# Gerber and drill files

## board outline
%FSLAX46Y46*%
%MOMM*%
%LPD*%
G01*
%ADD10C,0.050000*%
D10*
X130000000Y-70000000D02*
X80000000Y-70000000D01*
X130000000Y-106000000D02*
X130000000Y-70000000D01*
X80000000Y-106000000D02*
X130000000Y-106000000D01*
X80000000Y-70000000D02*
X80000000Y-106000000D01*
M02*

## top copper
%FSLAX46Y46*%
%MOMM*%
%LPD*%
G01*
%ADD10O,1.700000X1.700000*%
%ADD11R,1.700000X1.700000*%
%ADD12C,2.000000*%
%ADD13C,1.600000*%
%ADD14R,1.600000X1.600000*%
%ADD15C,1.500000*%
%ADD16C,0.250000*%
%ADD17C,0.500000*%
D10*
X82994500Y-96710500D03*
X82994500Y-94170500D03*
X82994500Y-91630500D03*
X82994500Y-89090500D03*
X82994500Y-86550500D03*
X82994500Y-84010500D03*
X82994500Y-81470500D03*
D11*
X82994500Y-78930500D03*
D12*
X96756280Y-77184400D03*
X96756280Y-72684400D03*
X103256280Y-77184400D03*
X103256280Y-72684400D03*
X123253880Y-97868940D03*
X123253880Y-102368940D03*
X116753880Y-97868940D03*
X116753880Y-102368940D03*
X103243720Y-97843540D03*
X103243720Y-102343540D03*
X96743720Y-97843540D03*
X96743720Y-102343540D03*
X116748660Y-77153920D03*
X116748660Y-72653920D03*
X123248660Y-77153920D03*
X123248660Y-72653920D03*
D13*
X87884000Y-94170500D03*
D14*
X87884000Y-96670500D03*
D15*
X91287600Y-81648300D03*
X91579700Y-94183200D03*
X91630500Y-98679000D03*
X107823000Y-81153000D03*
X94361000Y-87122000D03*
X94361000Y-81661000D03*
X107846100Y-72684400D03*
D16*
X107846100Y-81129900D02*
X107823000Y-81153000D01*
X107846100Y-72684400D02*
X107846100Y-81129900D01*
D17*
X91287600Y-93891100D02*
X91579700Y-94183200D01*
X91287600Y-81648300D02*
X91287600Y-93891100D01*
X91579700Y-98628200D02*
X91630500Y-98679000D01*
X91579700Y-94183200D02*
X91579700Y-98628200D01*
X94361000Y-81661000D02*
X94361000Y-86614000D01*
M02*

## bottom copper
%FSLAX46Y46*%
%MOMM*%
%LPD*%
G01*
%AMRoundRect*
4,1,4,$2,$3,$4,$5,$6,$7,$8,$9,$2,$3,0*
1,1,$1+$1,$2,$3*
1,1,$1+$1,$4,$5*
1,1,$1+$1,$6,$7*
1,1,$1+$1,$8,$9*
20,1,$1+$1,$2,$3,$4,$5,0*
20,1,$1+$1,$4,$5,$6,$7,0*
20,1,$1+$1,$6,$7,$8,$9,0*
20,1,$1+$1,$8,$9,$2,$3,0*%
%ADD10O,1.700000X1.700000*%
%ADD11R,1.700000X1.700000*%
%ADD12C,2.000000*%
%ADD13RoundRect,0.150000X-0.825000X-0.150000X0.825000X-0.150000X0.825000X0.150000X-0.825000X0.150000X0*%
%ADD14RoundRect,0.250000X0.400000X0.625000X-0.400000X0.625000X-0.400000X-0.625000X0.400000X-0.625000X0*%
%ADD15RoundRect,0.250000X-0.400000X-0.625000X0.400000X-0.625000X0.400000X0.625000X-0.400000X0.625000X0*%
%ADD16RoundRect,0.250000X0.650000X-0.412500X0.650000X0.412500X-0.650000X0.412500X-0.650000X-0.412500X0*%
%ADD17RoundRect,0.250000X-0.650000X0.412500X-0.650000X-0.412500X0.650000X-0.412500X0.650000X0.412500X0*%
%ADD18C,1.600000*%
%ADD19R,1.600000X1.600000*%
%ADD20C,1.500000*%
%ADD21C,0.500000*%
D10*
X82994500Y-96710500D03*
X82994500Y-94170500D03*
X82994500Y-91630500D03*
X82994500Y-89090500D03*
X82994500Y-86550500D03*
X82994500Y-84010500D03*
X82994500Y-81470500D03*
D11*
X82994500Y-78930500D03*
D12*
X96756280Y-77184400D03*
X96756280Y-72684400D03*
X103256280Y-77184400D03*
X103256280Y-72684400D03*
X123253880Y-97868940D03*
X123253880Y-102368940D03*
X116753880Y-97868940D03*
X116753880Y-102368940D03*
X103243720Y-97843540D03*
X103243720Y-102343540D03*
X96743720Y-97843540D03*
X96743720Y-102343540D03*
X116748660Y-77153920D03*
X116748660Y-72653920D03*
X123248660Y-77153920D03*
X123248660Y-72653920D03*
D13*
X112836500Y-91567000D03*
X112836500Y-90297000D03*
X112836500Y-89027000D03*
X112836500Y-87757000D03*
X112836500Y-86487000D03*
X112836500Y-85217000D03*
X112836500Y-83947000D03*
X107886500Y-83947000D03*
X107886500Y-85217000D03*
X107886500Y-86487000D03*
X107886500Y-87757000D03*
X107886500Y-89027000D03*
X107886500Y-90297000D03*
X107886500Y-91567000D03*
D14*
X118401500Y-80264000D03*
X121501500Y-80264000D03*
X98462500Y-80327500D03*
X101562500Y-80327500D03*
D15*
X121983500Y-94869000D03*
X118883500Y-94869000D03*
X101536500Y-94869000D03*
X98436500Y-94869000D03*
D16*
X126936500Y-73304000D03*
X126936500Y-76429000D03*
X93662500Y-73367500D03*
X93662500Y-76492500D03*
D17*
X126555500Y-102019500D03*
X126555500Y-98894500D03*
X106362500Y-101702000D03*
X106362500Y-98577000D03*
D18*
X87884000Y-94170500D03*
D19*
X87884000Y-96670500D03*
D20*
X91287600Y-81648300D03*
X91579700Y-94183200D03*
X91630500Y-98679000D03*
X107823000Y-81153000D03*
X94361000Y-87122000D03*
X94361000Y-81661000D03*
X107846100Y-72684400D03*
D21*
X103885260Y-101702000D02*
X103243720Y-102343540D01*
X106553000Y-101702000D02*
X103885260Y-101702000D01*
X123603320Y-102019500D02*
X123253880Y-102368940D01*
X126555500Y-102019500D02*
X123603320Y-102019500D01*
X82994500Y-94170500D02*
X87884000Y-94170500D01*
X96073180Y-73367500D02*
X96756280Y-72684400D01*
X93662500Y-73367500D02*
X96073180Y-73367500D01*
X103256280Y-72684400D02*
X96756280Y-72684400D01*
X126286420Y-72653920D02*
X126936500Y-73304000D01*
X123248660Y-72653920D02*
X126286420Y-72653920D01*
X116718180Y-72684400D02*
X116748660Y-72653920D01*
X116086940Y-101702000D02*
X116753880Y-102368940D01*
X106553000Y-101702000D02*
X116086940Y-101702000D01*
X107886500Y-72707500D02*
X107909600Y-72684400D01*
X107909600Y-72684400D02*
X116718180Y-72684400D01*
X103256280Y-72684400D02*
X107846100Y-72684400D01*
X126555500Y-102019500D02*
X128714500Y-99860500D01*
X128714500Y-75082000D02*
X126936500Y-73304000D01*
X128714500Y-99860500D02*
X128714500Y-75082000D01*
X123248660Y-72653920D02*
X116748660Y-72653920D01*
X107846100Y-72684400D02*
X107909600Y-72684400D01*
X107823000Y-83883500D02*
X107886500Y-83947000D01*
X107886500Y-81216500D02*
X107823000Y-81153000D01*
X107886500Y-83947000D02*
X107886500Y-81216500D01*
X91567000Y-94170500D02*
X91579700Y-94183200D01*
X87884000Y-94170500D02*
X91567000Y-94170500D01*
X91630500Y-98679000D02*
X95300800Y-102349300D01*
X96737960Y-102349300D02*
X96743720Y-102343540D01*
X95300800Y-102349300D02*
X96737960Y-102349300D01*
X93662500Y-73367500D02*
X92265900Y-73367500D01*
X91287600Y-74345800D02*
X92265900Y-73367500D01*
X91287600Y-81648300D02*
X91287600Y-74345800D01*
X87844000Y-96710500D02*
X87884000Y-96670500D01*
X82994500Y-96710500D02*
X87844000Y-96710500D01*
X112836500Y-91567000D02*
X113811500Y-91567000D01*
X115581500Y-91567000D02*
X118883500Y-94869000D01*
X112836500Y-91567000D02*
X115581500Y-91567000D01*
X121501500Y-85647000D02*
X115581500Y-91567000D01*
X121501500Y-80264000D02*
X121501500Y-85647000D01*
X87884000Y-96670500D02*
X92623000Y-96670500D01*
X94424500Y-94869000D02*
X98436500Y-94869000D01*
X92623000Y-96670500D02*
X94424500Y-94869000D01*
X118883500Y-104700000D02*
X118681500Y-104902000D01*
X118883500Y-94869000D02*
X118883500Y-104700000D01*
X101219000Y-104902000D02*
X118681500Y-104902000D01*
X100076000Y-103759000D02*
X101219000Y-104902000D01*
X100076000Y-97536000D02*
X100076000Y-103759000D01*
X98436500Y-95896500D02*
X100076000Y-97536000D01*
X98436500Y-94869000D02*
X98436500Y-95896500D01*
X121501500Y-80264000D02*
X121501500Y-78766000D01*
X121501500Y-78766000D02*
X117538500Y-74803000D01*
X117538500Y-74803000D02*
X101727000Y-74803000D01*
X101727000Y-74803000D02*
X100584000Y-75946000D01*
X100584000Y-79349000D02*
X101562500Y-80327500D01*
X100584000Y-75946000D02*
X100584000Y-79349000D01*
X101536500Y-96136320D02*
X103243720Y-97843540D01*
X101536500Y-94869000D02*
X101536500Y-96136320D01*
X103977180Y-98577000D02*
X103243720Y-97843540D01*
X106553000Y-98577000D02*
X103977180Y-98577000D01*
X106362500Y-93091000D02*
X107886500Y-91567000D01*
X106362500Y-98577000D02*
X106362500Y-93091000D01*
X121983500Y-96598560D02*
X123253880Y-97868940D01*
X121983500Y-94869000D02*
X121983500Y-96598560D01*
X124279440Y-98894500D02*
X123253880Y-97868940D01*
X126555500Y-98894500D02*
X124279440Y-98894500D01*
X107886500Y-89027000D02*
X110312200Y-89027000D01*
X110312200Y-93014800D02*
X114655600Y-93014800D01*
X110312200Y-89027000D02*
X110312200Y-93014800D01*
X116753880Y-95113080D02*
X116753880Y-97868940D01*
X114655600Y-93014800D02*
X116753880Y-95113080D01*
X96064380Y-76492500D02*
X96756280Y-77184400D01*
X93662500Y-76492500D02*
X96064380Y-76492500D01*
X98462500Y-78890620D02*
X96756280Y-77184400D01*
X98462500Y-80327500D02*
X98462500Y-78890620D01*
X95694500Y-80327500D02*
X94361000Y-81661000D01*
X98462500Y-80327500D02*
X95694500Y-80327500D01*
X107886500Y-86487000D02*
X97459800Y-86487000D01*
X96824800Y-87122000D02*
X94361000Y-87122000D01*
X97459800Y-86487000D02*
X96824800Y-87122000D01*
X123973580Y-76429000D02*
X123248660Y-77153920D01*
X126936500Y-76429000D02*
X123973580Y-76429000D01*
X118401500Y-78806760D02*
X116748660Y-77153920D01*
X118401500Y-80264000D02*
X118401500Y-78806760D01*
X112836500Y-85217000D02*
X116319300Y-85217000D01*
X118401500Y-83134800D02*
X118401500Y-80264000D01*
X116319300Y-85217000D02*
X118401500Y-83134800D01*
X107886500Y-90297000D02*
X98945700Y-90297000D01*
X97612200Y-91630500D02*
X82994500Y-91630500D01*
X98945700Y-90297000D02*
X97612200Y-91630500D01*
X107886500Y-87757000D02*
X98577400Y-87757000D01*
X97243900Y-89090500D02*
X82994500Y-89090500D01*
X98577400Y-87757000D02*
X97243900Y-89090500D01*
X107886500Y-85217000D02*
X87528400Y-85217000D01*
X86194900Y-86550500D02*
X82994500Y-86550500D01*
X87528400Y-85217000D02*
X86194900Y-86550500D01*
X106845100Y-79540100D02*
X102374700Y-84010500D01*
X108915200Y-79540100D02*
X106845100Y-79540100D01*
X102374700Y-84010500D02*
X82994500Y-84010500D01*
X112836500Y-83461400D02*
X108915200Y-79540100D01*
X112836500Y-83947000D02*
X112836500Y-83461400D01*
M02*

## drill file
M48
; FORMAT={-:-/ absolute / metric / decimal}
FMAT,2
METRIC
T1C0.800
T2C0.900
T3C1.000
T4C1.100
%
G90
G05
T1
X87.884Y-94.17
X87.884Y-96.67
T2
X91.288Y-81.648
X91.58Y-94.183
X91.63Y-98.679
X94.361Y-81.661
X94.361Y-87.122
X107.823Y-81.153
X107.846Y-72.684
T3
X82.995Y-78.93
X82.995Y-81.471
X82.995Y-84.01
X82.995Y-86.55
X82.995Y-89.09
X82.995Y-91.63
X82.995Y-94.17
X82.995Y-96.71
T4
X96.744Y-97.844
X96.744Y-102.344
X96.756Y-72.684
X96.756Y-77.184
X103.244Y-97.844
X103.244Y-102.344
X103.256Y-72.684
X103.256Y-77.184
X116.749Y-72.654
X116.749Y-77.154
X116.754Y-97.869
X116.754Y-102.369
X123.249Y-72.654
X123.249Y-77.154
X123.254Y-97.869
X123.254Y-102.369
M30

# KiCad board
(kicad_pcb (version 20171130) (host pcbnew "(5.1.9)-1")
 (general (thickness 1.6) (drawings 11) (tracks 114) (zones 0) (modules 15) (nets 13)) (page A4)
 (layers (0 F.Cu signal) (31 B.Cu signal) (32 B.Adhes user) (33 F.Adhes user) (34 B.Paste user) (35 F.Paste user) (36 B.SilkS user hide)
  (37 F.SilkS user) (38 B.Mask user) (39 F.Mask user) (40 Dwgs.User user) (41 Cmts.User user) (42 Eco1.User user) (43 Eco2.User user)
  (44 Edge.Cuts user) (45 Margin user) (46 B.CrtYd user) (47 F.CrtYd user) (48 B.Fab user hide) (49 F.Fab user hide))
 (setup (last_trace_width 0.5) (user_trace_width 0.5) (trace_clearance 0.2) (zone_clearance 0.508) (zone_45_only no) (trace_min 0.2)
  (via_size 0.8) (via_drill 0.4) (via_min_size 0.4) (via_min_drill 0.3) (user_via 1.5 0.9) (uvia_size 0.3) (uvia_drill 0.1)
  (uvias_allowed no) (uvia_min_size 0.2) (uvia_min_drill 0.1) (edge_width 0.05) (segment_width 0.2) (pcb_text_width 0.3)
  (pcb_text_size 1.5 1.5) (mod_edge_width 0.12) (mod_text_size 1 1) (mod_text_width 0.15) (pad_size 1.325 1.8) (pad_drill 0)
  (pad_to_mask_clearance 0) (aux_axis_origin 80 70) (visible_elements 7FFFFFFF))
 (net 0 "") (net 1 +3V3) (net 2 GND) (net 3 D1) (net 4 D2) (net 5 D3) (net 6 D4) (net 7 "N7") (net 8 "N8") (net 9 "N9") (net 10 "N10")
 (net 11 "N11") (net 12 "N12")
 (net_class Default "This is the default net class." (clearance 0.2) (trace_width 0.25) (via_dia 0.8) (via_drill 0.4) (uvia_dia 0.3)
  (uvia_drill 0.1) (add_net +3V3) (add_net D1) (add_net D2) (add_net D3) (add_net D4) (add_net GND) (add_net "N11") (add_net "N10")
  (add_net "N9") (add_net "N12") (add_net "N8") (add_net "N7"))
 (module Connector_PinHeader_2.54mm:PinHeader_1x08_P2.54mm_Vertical (layer F.Cu) (at 82.9945 78.9305)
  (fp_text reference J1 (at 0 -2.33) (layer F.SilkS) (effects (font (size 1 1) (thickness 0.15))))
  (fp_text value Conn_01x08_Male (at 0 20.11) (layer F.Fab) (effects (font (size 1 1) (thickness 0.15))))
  (pad 8 thru_hole oval (at 0 17.78) (size 1.7 1.7) (drill 1) (layers *.Cu *.Mask) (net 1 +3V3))
  (pad 7 thru_hole oval (at 0 15.24) (size 1.7 1.7) (drill 1) (layers *.Cu *.Mask) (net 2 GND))
  (pad 6 thru_hole oval (at 0 12.7) (size 1.7 1.7) (drill 1) (layers *.Cu *.Mask) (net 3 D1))
  (pad 5 thru_hole oval (at 0 10.16) (size 1.7 1.7) (drill 1) (layers *.Cu *.Mask) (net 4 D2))
  (pad 4 thru_hole oval (at 0 7.62) (size 1.7 1.7) (drill 1) (layers *.Cu *.Mask) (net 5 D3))
  (pad 3 thru_hole oval (at 0 5.08) (size 1.7 1.7) (drill 1) (layers *.Cu *.Mask) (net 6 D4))
  (pad 2 thru_hole oval (at 0 2.54) (size 1.7 1.7) (drill 1) (layers *.Cu *.Mask) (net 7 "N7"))
  (pad 1 thru_hole rect (at 0 0) (size 1.7 1.7) (drill 1) (layers *.Cu *.Mask) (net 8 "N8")))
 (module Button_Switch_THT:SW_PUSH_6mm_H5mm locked (layer F.Cu) (at 100 75 180)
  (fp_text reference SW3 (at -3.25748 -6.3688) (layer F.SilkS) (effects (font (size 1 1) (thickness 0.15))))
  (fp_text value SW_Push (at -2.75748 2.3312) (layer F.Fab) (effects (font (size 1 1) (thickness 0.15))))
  (pad 1 thru_hole circle (at 3.24372 -2.1844 270) (size 2 2) (drill 1.1) (layers *.Cu *.Mask) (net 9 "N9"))
  (pad 2 thru_hole circle (at 3.24372 2.3156 270) (size 2 2) (drill 1.1) (layers *.Cu *.Mask) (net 2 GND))
  (pad 1 thru_hole circle (at -3.25628 -2.1844 270) (size 2 2) (drill 1.1) (layers *.Cu *.Mask) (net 9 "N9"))
  (pad 2 thru_hole circle (at -3.25628 2.3156 270) (size 2 2) (drill 1.1) (layers *.Cu *.Mask) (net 2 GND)))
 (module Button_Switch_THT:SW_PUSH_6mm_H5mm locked (layer F.Cu) (at 120 100)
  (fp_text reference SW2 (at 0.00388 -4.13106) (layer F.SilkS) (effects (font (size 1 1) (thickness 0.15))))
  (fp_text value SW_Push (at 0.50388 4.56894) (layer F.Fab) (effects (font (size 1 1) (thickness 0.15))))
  (pad 1 thru_hole circle (at 3.25388 -2.13106 90) (size 2 2) (drill 1.1) (layers *.Cu *.Mask) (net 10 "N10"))
  (pad 2 thru_hole circle (at 3.25388 2.36894 90) (size 2 2) (drill 1.1) (layers *.Cu *.Mask) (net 2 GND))
  (pad 1 thru_hole circle (at -3.24612 -2.13106 90) (size 2 2) (drill 1.1) (layers *.Cu *.Mask) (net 10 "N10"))
  (pad 2 thru_hole circle (at -3.24612 2.36894 90) (size 2 2) (drill 1.1) (layers *.Cu *.Mask) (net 2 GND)))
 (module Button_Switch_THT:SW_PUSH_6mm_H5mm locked (layer F.Cu) (at 100 100)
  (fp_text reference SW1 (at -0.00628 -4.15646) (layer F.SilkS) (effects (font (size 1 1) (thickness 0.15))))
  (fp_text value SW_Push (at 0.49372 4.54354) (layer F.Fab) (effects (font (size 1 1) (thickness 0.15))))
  (pad 1 thru_hole circle (at 3.24372 -2.15646 90) (size 2 2) (drill 1.1) (layers *.Cu *.Mask) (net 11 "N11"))
  (pad 2 thru_hole circle (at 3.24372 2.34354 90) (size 2 2) (drill 1.1) (layers *.Cu *.Mask) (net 2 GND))
  (pad 1 thru_hole circle (at -3.25628 -2.15646 90) (size 2 2) (drill 1.1) (layers *.Cu *.Mask) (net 11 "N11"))
  (pad 2 thru_hole circle (at -3.25628 2.34354 90) (size 2 2) (drill 1.1) (layers *.Cu *.Mask) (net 2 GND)))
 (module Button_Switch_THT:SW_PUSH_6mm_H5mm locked (layer F.Cu) (at 120 75 180)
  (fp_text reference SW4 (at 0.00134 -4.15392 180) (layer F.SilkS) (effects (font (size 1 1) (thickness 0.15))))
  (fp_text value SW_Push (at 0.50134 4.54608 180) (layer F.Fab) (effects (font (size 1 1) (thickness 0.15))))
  (pad 1 thru_hole circle (at 3.25134 -2.15392 270) (size 2 2) (drill 1.1) (layers *.Cu *.Mask) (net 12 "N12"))
  (pad 2 thru_hole circle (at 3.25134 2.34608 270) (size 2 2) (drill 1.1) (layers *.Cu *.Mask) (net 2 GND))
  (pad 1 thru_hole circle (at -3.24866 -2.15392 270) (size 2 2) (drill 1.1) (layers *.Cu *.Mask) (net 12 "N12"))
  (pad 2 thru_hole circle (at -3.24866 2.34608 270) (size 2 2) (drill 1.1) (layers *.Cu *.Mask) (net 2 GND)))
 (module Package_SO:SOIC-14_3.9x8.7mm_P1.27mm (layer B.Cu) (at 110.3615 87.757)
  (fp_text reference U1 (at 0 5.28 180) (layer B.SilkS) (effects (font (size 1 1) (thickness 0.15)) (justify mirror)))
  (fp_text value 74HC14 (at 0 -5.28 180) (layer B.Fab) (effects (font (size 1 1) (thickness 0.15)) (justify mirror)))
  (pad 14 smd roundrect (at 2.475 3.81) (size 1.95 0.6) (layers B.Cu B.Paste B.Mask) (roundrect_rratio 0.25) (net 1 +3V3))
  (pad 13 smd roundrect (at 2.475 2.54) (size 1.95 0.6) (layers B.Cu B.Paste B.Mask) (roundrect_rratio 0.25))
  (pad 12 smd roundrect (at 2.475 1.27) (size 1.95 0.6) (layers B.Cu B.Paste B.Mask) (roundrect_rratio 0.25))
  (pad 11 smd roundrect (at 2.475 0) (size 1.95 0.6) (layers B.Cu B.Paste B.Mask) (roundrect_rratio 0.25))
  (pad 10 smd roundrect (at 2.475 -1.27) (size 1.95 0.6) (layers B.Cu B.Paste B.Mask) (roundrect_rratio 0.25))
  (pad 9 smd roundrect (at 2.475 -2.54) (size 1.95 0.6) (layers B.Cu B.Paste B.Mask) (roundrect_rratio 0.25) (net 12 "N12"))
  (pad 8 smd roundrect (at 2.475 -3.81) (size 1.95 0.6) (layers B.Cu B.Paste B.Mask) (roundrect_rratio 0.25) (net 6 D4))
  (pad 7 smd roundrect (at -2.475 -3.81) (size 1.95 0.6) (layers B.Cu B.Paste B.Mask) (roundrect_rratio 0.25) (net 2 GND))
  (pad 6 smd roundrect (at -2.475 -2.54) (size 1.95 0.6) (layers B.Cu B.Paste B.Mask) (roundrect_rratio 0.25) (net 5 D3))
  (pad 5 smd roundrect (at -2.475 -1.27) (size 1.95 0.6) (layers B.Cu B.Paste B.Mask) (roundrect_rratio 0.25) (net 9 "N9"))
  (pad 4 smd roundrect (at -2.475 0) (size 1.95 0.6) (layers B.Cu B.Paste B.Mask) (roundrect_rratio 0.25) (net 4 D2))
  (pad 3 smd roundrect (at -2.475 1.27) (size 1.95 0.6) (layers B.Cu B.Paste B.Mask) (roundrect_rratio 0.25) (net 10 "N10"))
  (pad 2 smd roundrect (at -2.475 2.54) (size 1.95 0.6) (layers B.Cu B.Paste B.Mask) (roundrect_rratio 0.25) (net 3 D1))
  (pad 1 smd roundrect (at -2.475 3.81) (size 1.95 0.6) (layers B.Cu B.Paste B.Mask) (roundrect_rratio 0.25) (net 11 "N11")))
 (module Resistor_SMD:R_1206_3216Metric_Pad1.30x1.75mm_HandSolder (layer B.Cu) (at 119.9515 80.264 180)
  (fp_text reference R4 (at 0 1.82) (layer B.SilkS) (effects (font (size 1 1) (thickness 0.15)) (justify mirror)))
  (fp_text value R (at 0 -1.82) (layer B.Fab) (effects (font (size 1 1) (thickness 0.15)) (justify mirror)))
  (pad 2 smd roundrect (at 1.55 0 180) (size 1.3 1.75) (layers B.Cu B.Paste B.Mask) (roundrect_rratio 0.192308) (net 12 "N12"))
  (pad 1 smd roundrect (at -1.55 0 180) (size 1.3 1.75) (layers B.Cu B.Paste B.Mask) (roundrect_rratio 0.192308) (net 1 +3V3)))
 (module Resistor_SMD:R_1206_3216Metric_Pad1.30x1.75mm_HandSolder (layer B.Cu) (at 100.0125 80.3275 180)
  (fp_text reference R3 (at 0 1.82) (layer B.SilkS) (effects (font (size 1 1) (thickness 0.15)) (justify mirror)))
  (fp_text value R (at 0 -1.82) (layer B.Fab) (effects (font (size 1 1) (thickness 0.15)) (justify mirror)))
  (pad 2 smd roundrect (at 1.55 0 180) (size 1.3 1.75) (layers B.Cu B.Paste B.Mask) (roundrect_rratio 0.192308) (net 9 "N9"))
  (pad 1 smd roundrect (at -1.55 0 180) (size 1.3 1.75) (layers B.Cu B.Paste B.Mask) (roundrect_rratio 0.192308) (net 1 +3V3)))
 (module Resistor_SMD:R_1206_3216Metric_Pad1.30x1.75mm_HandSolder (layer B.Cu) (at 120.4335 94.869)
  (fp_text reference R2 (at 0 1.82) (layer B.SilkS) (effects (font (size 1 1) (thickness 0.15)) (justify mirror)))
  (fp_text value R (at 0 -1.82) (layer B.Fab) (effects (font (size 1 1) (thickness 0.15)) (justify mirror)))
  (pad 2 smd roundrect (at 1.55 0) (size 1.3 1.75) (layers B.Cu B.Paste B.Mask) (roundrect_rratio 0.192308) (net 10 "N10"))
  (pad 1 smd roundrect (at -1.55 0) (size 1.3 1.75) (layers B.Cu B.Paste B.Mask) (roundrect_rratio 0.192308) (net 1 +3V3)))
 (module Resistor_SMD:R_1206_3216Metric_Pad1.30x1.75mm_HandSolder (layer B.Cu) (at 99.9865 94.869)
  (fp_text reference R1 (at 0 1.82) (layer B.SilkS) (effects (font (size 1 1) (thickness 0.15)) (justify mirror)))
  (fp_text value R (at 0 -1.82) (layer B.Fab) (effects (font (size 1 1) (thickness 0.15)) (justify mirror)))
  (pad 2 smd roundrect (at 1.55 0) (size 1.3 1.75) (layers B.Cu B.Paste B.Mask) (roundrect_rratio 0.192308) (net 11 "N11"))
  (pad 1 smd roundrect (at -1.55 0) (size 1.3 1.75) (layers B.Cu B.Paste B.Mask) (roundrect_rratio 0.192308) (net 1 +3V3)))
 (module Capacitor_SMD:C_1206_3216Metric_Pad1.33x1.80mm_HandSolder (layer B.Cu) (at 126.9365 74.8665 90)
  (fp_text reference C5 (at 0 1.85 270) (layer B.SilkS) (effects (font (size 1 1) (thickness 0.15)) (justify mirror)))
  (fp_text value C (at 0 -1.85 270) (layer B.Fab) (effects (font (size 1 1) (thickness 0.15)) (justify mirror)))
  (pad 2 smd roundrect (at 1.5625 0 90) (size 1.325 1.8) (layers B.Cu B.Paste B.Mask) (roundrect_rratio 0.188679) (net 2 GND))
  (pad 1 smd roundrect (at -1.5625 0 90) (size 1.325 1.8) (layers B.Cu B.Paste B.Mask) (roundrect_rratio 0.188679) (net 12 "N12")))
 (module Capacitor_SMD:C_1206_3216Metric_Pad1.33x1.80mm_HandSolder (layer B.Cu) (at 93.6625 74.93 90)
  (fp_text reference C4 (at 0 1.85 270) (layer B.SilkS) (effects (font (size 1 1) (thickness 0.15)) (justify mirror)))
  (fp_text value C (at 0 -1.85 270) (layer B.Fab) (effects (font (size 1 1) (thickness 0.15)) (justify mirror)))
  (pad 2 smd roundrect (at 1.5625 0 90) (size 1.325 1.8) (layers B.Cu B.Paste B.Mask) (roundrect_rratio 0.188679) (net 2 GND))
  (pad 1 smd roundrect (at -1.5625 0 90) (size 1.325 1.8) (layers B.Cu B.Paste B.Mask) (roundrect_rratio 0.188679) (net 9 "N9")))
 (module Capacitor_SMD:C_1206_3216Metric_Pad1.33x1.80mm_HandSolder (layer B.Cu) (at 126.5555 100.457 270)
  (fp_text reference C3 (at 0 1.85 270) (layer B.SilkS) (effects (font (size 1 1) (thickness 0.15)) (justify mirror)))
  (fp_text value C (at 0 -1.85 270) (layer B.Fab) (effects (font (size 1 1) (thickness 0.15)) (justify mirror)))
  (pad 2 smd roundrect (at 1.5625 0 270) (size 1.325 1.8) (layers B.Cu B.Paste B.Mask) (roundrect_rratio 0.188679) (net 2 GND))
  (pad 1 smd roundrect (at -1.5625 0 270) (size 1.325 1.8) (layers B.Cu B.Paste B.Mask) (roundrect_rratio 0.188679) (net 10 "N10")))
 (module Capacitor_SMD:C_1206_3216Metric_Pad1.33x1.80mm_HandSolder (layer B.Cu) (at 106.3625 100.1395 270)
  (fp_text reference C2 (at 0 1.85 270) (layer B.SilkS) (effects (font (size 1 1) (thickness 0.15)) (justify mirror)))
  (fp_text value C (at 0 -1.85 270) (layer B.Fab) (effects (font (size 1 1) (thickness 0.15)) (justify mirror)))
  (pad 2 smd roundrect (at 1.5625 0 270) (size 1.325 1.8) (layers B.Cu B.Paste B.Mask) (roundrect_rratio 0.188679) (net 2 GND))
  (pad 1 smd roundrect (at -1.5625 0 270) (size 1.325 1.8) (layers B.Cu B.Paste B.Mask) (roundrect_rratio 0.188679) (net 11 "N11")))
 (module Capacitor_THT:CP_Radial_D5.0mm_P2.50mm (layer F.Cu) (at 87.884 96.6705 90)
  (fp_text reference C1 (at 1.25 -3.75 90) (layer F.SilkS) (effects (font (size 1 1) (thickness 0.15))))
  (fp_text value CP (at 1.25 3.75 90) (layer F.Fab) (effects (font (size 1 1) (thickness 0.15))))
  (pad 2 thru_hole circle (at 2.5 0 90) (size 1.6 1.6) (drill 0.8) (layers *.Cu *.Mask) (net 2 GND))
  (pad 1 thru_hole rect (at 0 0 90) (size 1.6 1.6) (drill 0.8) (layers *.Cu *.Mask) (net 1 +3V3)))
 (gr_line (start 130 70) (end 80 70) (layer Edge.Cuts) (width 0.05))
 (gr_line (start 130 106) (end 130 70) (layer Edge.Cuts) (width 0.05))
 (gr_line (start 80 106) (end 130 106) (layer Edge.Cuts) (width 0.05))
 (gr_line (start 80 70) (end 80 106) (layer Edge.Cuts) (width 0.05))
 (via (at 91.2876 81.6483) (size 1.5) (drill 0.9) (layers F.Cu B.Cu) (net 2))
 (via (at 91.5797 94.1832) (size 1.5) (drill 0.9) (layers F.Cu B.Cu) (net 2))
 (via (at 91.6305 98.679) (size 1.5) (drill 0.9) (layers F.Cu B.Cu) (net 2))
 (via (at 107.823 81.153) (size 1.5) (drill 0.9) (layers F.Cu B.Cu) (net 2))
 (via (at 94.361 87.122) (size 1.5) (drill 0.9) (layers F.Cu B.Cu) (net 9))
 (via (at 94.361 81.661) (size 1.5) (drill 0.9) (layers F.Cu B.Cu) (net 9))
 (segment (start 103.88526 101.702) (end 103.24372 102.34354) (width 0.5) (layer B.Cu) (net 2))
 (segment (start 106.553 101.702) (end 103.88526 101.702) (width 0.5) (layer B.Cu) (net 2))
 (segment (start 123.60332 102.0195) (end 123.25388 102.36894) (width 0.5) (layer B.Cu) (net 2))
 (segment (start 126.5555 102.0195) (end 123.60332 102.0195) (width 0.5) (layer B.Cu) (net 2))
 (segment (start 82.9945 94.1705) (end 87.884 94.1705) (width 0.5) (layer B.Cu) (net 2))
 (segment (start 96.07318 73.3675) (end 96.75628 72.6844) (width 0.5) (layer B.Cu) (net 2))
 (segment (start 93.6625 73.3675) (end 96.07318 73.3675) (width 0.5) (layer B.Cu) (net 2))
 (segment (start 103.25628 72.6844) (end 96.75628 72.6844) (width 0.5) (layer B.Cu) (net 2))
 (segment (start 126.28642 72.65392) (end 126.9365 73.304) (width 0.5) (layer B.Cu) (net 2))
 (segment (start 123.24866 72.65392) (end 126.28642 72.65392) (width 0.5) (layer B.Cu) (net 2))
 (segment (start 116.71818 72.6844) (end 116.74866 72.65392) (width 0.5) (layer B.Cu) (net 2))
 (segment (start 116.08694 101.702) (end 116.75388 102.36894) (width 0.5) (layer B.Cu) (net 2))
 (segment (start 106.553 101.702) (end 116.08694 101.702) (width 0.5) (layer B.Cu) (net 2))
 (segment (start 107.8865 72.7075) (end 107.9096 72.6844) (width 0.5) (layer B.Cu) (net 2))
 (segment (start 107.9096 72.6844) (end 116.71818 72.6844) (width 0.5) (layer B.Cu) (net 2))
 (segment (start 103.25628 72.6844) (end 107.8461 72.6844) (width 0.5) (layer B.Cu) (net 2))
 (segment (start 126.5555 102.0195) (end 128.7145 99.8605) (width 0.5) (layer B.Cu) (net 2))
 (segment (start 128.7145 75.082) (end 126.9365 73.304) (width 0.5) (layer B.Cu) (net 2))
 (segment (start 128.7145 99.8605) (end 128.7145 75.082) (width 0.5) (layer B.Cu) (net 2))
 (segment (start 123.24866 72.65392) (end 116.74866 72.65392) (width 0.5) (layer B.Cu) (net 2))
 (segment (start 107.8461 72.6844) (end 107.9096 72.6844) (width 0.5) (layer B.Cu) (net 2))
 (via (at 107.8461 72.6844) (size 1.5) (drill 0.9) (layers F.Cu B.Cu) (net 2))
 (segment (start 107.823 83.8835) (end 107.8865 83.947) (width 0.5) (layer B.Cu) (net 2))
 (segment (start 107.8865 81.2165) (end 107.823 81.153) (width 0.5) (layer B.Cu) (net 2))
 (segment (start 107.8865 83.947) (end 107.8865 81.2165) (width 0.5) (layer B.Cu) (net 2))
 (segment (start 107.8461 81.1299) (end 107.823 81.153) (width 0.25) (layer F.Cu) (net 2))
 (segment (start 107.8461 72.6844) (end 107.8461 81.1299) (width 0.25) (layer F.Cu) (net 2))
 (segment (start 91.567 94.1705) (end 91.5797 94.1832) (width 0.5) (layer B.Cu) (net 2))
 (segment (start 87.884 94.1705) (end 91.567 94.1705) (width 0.5) (layer B.Cu) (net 2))
 (segment (start 91.6305 98.679) (end 95.3008 102.3493) (width 0.5) (layer B.Cu) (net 2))
 (segment (start 96.73796 102.3493) (end 96.74372 102.34354) (width 0.5) (layer B.Cu) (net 2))
 (segment (start 95.3008 102.3493) (end 96.73796 102.3493) (width 0.5) (layer B.Cu) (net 2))
 (segment (start 93.6625 73.3675) (end 92.2659 73.3675) (width 0.5) (layer B.Cu) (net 2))
 (segment (start 91.2876 74.3458) (end 92.2659 73.3675) (width 0.5) (layer B.Cu) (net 2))
 (segment (start 91.2876 81.6483) (end 91.2876 74.3458) (width 0.5) (layer B.Cu) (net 2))
 (segment (start 91.2876 93.8911) (end 91.5797 94.1832) (width 0.5) (layer F.Cu) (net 2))
 (segment (start 91.2876 81.6483) (end 91.2876 93.8911) (width 0.5) (layer F.Cu) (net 2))
 (segment (start 91.5797 98.6282) (end 91.6305 98.679) (width 0.5) (layer F.Cu) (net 2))
 (segment (start 91.5797 94.1832) (end 91.5797 98.6282) (width 0.5) (layer F.Cu) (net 2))
 (segment (start 87.844 96.7105) (end 87.884 96.6705) (width 0.5) (layer B.Cu) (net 1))
 (segment (start 82.9945 96.7105) (end 87.844 96.7105) (width 0.5) (layer B.Cu) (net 1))
 (segment (start 112.8365 91.567) (end 113.8115 91.567) (width 0.5) (layer B.Cu) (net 1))
 (segment (start 115.5815 91.567) (end 118.8835 94.869) (width 0.5) (layer B.Cu) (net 1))
 (segment (start 112.8365 91.567) (end 115.5815 91.567) (width 0.5) (layer B.Cu) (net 1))
 (segment (start 121.5015 85.647) (end 115.5815 91.567) (width 0.5) (layer B.Cu) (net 1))
 (segment (start 121.5015 80.264) (end 121.5015 85.647) (width 0.5) (layer B.Cu) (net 1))
 (segment (start 87.884 96.6705) (end 92.623 96.6705) (width 0.5) (layer B.Cu) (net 1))
 (segment (start 94.4245 94.869) (end 98.4365 94.869) (width 0.5) (layer B.Cu) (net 1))
 (segment (start 92.623 96.6705) (end 94.4245 94.869) (width 0.5) (layer B.Cu) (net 1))
 (segment (start 118.8835 104.7) (end 118.6815 104.902) (width 0.5) (layer B.Cu) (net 1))
 (segment (start 118.8835 94.869) (end 118.8835 104.7) (width 0.5) (layer B.Cu) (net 1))
 (segment (start 101.219 104.902) (end 118.6815 104.902) (width 0.5) (layer B.Cu) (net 1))
 (segment (start 100.076 103.759) (end 101.219 104.902) (width 0.5) (layer B.Cu) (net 1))
 (segment (start 100.076 97.536) (end 100.076 103.759) (width 0.5) (layer B.Cu) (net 1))
 (segment (start 98.4365 95.8965) (end 100.076 97.536) (width 0.5) (layer B.Cu) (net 1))
 (segment (start 98.4365 94.869) (end 98.4365 95.8965) (width 0.5) (layer B.Cu) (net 1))
 (segment (start 121.5015 80.264) (end 121.5015 78.766) (width 0.5) (layer B.Cu) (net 1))
 (segment (start 121.5015 78.766) (end 117.5385 74.803) (width 0.5) (layer B.Cu) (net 1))
 (segment (start 117.5385 74.803) (end 101.727 74.803) (width 0.5) (layer B.Cu) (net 1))
 (segment (start 101.727 74.803) (end 100.584 75.946) (width 0.5) (layer B.Cu) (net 1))
 (segment (start 100.584 79.349) (end 101.5625 80.3275) (width 0.5) (layer B.Cu) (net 1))
 (segment (start 100.584 75.946) (end 100.584 79.349) (width 0.5) (layer B.Cu) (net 1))
 (segment (start 101.5365 96.13632) (end 103.24372 97.84354) (width 0.5) (layer B.Cu) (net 11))
 (segment (start 101.5365 94.869) (end 101.5365 96.13632) (width 0.5) (layer B.Cu) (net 11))
 (segment (start 103.97718 98.577) (end 103.24372 97.84354) (width 0.5) (layer B.Cu) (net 11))
 (segment (start 106.553 98.577) (end 103.97718 98.577) (width 0.5) (layer B.Cu) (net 11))
 (segment (start 106.3625 93.091) (end 107.8865 91.567) (width 0.5) (layer B.Cu) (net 11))
 (segment (start 106.3625 98.577) (end 106.3625 93.091) (width 0.5) (layer B.Cu) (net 11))
 (segment (start 121.9835 96.59856) (end 123.25388 97.86894) (width 0.5) (layer B.Cu) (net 10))
 (segment (start 121.9835 94.869) (end 121.9835 96.59856) (width 0.5) (layer B.Cu) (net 10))
 (segment (start 124.27944 98.8945) (end 123.25388 97.86894) (width 0.5) (layer B.Cu) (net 10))
 (segment (start 126.5555 98.8945) (end 124.27944 98.8945) (width 0.5) (layer B.Cu) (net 10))
 (segment (start 107.8865 89.027) (end 110.3122 89.027) (width 0.5) (layer B.Cu) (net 10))
 (segment (start 110.3122 93.0148) (end 114.6556 93.0148) (width 0.5) (layer B.Cu) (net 10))
 (segment (start 110.3122 89.027) (end 110.3122 93.0148) (width 0.5) (layer B.Cu) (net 10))
 (segment (start 116.75388 95.11308) (end 116.75388 97.86894) (width 0.5) (layer B.Cu) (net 10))
 (segment (start 114.6556 93.0148) (end 116.75388 95.11308) (width 0.5) (layer B.Cu) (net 10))
 (segment (start 96.06438 76.4925) (end 96.75628 77.1844) (width 0.5) (layer B.Cu) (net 9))
 (segment (start 93.6625 76.4925) (end 96.06438 76.4925) (width 0.5) (layer B.Cu) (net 9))
 (segment (start 98.4625 78.89062) (end 96.75628 77.1844) (width 0.5) (layer B.Cu) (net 9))
 (segment (start 98.4625 80.3275) (end 98.4625 78.89062) (width 0.5) (layer B.Cu) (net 9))
 (segment (start 95.6945 80.3275) (end 94.361 81.661) (width 0.5) (layer B.Cu) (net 9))
 (segment (start 98.4625 80.3275) (end 95.6945 80.3275) (width 0.5) (layer B.Cu) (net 9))
 (segment (start 94.361 81.661) (end 94.361 86.614) (width 0.5) (layer F.Cu) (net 9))
 (segment (start 107.8865 86.487) (end 97.4598 86.487) (width 0.5) (layer B.Cu) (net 9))
 (segment (start 96.8248 87.122) (end 94.361 87.122) (width 0.5) (layer B.Cu) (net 9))
 (segment (start 97.4598 86.487) (end 96.8248 87.122) (width 0.5) (layer B.Cu) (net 9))
 (segment (start 123.97358 76.429) (end 123.24866 77.15392) (width 0.5) (layer B.Cu) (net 12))
 (segment (start 126.9365 76.429) (end 123.97358 76.429) (width 0.5) (layer B.Cu) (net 12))
 (segment (start 118.4015 78.80676) (end 116.74866 77.15392) (width 0.5) (layer B.Cu) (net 12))
 (segment (start 118.4015 80.264) (end 118.4015 78.80676) (width 0.5) (layer B.Cu) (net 12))
 (segment (start 112.8365 85.217) (end 116.3193 85.217) (width 0.5) (layer B.Cu) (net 12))
 (segment (start 118.4015 83.1348) (end 118.4015 80.264) (width 0.5) (layer B.Cu) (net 12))
 (segment (start 116.3193 85.217) (end 118.4015 83.1348) (width 0.5) (layer B.Cu) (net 12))
 (segment (start 107.8865 90.297) (end 98.9457 90.297) (width 0.5) (layer B.Cu) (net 3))
 (segment (start 97.6122 91.6305) (end 82.9945 91.6305) (width 0.5) (layer B.Cu) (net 3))
 (segment (start 98.9457 90.297) (end 97.6122 91.6305) (width 0.5) (layer B.Cu) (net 3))
 (segment (start 107.8865 87.757) (end 98.5774 87.757) (width 0.5) (layer B.Cu) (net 4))
 (segment (start 97.2439 89.0905) (end 82.9945 89.0905) (width 0.5) (layer B.Cu) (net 4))
 (segment (start 98.5774 87.757) (end 97.2439 89.0905) (width 0.5) (layer B.Cu) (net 4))
 (segment (start 107.8865 85.217) (end 87.5284 85.217) (width 0.5) (layer B.Cu) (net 5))
 (segment (start 86.1949 86.5505) (end 82.9945 86.5505) (width 0.5) (layer B.Cu) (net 5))
 (segment (start 87.5284 85.217) (end 86.1949 86.5505) (width 0.5) (layer B.Cu) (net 5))
 (segment (start 106.8451 79.5401) (end 102.3747 84.0105) (width 0.5) (layer B.Cu) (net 6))
 (segment (start 108.9152 79.5401) (end 106.8451 79.5401) (width 0.5) (layer B.Cu) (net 6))
 (segment (start 102.3747 84.0105) (end 82.9945 84.0105) (width 0.5) (layer B.Cu) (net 6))
 (segment (start 112.8365 83.4614) (end 108.9152 79.5401) (width 0.5) (layer B.Cu) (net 6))
 (segment (start 112.8365 83.947) (end 112.8365 83.4614) (width 0.5) (layer B.Cu) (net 6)))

